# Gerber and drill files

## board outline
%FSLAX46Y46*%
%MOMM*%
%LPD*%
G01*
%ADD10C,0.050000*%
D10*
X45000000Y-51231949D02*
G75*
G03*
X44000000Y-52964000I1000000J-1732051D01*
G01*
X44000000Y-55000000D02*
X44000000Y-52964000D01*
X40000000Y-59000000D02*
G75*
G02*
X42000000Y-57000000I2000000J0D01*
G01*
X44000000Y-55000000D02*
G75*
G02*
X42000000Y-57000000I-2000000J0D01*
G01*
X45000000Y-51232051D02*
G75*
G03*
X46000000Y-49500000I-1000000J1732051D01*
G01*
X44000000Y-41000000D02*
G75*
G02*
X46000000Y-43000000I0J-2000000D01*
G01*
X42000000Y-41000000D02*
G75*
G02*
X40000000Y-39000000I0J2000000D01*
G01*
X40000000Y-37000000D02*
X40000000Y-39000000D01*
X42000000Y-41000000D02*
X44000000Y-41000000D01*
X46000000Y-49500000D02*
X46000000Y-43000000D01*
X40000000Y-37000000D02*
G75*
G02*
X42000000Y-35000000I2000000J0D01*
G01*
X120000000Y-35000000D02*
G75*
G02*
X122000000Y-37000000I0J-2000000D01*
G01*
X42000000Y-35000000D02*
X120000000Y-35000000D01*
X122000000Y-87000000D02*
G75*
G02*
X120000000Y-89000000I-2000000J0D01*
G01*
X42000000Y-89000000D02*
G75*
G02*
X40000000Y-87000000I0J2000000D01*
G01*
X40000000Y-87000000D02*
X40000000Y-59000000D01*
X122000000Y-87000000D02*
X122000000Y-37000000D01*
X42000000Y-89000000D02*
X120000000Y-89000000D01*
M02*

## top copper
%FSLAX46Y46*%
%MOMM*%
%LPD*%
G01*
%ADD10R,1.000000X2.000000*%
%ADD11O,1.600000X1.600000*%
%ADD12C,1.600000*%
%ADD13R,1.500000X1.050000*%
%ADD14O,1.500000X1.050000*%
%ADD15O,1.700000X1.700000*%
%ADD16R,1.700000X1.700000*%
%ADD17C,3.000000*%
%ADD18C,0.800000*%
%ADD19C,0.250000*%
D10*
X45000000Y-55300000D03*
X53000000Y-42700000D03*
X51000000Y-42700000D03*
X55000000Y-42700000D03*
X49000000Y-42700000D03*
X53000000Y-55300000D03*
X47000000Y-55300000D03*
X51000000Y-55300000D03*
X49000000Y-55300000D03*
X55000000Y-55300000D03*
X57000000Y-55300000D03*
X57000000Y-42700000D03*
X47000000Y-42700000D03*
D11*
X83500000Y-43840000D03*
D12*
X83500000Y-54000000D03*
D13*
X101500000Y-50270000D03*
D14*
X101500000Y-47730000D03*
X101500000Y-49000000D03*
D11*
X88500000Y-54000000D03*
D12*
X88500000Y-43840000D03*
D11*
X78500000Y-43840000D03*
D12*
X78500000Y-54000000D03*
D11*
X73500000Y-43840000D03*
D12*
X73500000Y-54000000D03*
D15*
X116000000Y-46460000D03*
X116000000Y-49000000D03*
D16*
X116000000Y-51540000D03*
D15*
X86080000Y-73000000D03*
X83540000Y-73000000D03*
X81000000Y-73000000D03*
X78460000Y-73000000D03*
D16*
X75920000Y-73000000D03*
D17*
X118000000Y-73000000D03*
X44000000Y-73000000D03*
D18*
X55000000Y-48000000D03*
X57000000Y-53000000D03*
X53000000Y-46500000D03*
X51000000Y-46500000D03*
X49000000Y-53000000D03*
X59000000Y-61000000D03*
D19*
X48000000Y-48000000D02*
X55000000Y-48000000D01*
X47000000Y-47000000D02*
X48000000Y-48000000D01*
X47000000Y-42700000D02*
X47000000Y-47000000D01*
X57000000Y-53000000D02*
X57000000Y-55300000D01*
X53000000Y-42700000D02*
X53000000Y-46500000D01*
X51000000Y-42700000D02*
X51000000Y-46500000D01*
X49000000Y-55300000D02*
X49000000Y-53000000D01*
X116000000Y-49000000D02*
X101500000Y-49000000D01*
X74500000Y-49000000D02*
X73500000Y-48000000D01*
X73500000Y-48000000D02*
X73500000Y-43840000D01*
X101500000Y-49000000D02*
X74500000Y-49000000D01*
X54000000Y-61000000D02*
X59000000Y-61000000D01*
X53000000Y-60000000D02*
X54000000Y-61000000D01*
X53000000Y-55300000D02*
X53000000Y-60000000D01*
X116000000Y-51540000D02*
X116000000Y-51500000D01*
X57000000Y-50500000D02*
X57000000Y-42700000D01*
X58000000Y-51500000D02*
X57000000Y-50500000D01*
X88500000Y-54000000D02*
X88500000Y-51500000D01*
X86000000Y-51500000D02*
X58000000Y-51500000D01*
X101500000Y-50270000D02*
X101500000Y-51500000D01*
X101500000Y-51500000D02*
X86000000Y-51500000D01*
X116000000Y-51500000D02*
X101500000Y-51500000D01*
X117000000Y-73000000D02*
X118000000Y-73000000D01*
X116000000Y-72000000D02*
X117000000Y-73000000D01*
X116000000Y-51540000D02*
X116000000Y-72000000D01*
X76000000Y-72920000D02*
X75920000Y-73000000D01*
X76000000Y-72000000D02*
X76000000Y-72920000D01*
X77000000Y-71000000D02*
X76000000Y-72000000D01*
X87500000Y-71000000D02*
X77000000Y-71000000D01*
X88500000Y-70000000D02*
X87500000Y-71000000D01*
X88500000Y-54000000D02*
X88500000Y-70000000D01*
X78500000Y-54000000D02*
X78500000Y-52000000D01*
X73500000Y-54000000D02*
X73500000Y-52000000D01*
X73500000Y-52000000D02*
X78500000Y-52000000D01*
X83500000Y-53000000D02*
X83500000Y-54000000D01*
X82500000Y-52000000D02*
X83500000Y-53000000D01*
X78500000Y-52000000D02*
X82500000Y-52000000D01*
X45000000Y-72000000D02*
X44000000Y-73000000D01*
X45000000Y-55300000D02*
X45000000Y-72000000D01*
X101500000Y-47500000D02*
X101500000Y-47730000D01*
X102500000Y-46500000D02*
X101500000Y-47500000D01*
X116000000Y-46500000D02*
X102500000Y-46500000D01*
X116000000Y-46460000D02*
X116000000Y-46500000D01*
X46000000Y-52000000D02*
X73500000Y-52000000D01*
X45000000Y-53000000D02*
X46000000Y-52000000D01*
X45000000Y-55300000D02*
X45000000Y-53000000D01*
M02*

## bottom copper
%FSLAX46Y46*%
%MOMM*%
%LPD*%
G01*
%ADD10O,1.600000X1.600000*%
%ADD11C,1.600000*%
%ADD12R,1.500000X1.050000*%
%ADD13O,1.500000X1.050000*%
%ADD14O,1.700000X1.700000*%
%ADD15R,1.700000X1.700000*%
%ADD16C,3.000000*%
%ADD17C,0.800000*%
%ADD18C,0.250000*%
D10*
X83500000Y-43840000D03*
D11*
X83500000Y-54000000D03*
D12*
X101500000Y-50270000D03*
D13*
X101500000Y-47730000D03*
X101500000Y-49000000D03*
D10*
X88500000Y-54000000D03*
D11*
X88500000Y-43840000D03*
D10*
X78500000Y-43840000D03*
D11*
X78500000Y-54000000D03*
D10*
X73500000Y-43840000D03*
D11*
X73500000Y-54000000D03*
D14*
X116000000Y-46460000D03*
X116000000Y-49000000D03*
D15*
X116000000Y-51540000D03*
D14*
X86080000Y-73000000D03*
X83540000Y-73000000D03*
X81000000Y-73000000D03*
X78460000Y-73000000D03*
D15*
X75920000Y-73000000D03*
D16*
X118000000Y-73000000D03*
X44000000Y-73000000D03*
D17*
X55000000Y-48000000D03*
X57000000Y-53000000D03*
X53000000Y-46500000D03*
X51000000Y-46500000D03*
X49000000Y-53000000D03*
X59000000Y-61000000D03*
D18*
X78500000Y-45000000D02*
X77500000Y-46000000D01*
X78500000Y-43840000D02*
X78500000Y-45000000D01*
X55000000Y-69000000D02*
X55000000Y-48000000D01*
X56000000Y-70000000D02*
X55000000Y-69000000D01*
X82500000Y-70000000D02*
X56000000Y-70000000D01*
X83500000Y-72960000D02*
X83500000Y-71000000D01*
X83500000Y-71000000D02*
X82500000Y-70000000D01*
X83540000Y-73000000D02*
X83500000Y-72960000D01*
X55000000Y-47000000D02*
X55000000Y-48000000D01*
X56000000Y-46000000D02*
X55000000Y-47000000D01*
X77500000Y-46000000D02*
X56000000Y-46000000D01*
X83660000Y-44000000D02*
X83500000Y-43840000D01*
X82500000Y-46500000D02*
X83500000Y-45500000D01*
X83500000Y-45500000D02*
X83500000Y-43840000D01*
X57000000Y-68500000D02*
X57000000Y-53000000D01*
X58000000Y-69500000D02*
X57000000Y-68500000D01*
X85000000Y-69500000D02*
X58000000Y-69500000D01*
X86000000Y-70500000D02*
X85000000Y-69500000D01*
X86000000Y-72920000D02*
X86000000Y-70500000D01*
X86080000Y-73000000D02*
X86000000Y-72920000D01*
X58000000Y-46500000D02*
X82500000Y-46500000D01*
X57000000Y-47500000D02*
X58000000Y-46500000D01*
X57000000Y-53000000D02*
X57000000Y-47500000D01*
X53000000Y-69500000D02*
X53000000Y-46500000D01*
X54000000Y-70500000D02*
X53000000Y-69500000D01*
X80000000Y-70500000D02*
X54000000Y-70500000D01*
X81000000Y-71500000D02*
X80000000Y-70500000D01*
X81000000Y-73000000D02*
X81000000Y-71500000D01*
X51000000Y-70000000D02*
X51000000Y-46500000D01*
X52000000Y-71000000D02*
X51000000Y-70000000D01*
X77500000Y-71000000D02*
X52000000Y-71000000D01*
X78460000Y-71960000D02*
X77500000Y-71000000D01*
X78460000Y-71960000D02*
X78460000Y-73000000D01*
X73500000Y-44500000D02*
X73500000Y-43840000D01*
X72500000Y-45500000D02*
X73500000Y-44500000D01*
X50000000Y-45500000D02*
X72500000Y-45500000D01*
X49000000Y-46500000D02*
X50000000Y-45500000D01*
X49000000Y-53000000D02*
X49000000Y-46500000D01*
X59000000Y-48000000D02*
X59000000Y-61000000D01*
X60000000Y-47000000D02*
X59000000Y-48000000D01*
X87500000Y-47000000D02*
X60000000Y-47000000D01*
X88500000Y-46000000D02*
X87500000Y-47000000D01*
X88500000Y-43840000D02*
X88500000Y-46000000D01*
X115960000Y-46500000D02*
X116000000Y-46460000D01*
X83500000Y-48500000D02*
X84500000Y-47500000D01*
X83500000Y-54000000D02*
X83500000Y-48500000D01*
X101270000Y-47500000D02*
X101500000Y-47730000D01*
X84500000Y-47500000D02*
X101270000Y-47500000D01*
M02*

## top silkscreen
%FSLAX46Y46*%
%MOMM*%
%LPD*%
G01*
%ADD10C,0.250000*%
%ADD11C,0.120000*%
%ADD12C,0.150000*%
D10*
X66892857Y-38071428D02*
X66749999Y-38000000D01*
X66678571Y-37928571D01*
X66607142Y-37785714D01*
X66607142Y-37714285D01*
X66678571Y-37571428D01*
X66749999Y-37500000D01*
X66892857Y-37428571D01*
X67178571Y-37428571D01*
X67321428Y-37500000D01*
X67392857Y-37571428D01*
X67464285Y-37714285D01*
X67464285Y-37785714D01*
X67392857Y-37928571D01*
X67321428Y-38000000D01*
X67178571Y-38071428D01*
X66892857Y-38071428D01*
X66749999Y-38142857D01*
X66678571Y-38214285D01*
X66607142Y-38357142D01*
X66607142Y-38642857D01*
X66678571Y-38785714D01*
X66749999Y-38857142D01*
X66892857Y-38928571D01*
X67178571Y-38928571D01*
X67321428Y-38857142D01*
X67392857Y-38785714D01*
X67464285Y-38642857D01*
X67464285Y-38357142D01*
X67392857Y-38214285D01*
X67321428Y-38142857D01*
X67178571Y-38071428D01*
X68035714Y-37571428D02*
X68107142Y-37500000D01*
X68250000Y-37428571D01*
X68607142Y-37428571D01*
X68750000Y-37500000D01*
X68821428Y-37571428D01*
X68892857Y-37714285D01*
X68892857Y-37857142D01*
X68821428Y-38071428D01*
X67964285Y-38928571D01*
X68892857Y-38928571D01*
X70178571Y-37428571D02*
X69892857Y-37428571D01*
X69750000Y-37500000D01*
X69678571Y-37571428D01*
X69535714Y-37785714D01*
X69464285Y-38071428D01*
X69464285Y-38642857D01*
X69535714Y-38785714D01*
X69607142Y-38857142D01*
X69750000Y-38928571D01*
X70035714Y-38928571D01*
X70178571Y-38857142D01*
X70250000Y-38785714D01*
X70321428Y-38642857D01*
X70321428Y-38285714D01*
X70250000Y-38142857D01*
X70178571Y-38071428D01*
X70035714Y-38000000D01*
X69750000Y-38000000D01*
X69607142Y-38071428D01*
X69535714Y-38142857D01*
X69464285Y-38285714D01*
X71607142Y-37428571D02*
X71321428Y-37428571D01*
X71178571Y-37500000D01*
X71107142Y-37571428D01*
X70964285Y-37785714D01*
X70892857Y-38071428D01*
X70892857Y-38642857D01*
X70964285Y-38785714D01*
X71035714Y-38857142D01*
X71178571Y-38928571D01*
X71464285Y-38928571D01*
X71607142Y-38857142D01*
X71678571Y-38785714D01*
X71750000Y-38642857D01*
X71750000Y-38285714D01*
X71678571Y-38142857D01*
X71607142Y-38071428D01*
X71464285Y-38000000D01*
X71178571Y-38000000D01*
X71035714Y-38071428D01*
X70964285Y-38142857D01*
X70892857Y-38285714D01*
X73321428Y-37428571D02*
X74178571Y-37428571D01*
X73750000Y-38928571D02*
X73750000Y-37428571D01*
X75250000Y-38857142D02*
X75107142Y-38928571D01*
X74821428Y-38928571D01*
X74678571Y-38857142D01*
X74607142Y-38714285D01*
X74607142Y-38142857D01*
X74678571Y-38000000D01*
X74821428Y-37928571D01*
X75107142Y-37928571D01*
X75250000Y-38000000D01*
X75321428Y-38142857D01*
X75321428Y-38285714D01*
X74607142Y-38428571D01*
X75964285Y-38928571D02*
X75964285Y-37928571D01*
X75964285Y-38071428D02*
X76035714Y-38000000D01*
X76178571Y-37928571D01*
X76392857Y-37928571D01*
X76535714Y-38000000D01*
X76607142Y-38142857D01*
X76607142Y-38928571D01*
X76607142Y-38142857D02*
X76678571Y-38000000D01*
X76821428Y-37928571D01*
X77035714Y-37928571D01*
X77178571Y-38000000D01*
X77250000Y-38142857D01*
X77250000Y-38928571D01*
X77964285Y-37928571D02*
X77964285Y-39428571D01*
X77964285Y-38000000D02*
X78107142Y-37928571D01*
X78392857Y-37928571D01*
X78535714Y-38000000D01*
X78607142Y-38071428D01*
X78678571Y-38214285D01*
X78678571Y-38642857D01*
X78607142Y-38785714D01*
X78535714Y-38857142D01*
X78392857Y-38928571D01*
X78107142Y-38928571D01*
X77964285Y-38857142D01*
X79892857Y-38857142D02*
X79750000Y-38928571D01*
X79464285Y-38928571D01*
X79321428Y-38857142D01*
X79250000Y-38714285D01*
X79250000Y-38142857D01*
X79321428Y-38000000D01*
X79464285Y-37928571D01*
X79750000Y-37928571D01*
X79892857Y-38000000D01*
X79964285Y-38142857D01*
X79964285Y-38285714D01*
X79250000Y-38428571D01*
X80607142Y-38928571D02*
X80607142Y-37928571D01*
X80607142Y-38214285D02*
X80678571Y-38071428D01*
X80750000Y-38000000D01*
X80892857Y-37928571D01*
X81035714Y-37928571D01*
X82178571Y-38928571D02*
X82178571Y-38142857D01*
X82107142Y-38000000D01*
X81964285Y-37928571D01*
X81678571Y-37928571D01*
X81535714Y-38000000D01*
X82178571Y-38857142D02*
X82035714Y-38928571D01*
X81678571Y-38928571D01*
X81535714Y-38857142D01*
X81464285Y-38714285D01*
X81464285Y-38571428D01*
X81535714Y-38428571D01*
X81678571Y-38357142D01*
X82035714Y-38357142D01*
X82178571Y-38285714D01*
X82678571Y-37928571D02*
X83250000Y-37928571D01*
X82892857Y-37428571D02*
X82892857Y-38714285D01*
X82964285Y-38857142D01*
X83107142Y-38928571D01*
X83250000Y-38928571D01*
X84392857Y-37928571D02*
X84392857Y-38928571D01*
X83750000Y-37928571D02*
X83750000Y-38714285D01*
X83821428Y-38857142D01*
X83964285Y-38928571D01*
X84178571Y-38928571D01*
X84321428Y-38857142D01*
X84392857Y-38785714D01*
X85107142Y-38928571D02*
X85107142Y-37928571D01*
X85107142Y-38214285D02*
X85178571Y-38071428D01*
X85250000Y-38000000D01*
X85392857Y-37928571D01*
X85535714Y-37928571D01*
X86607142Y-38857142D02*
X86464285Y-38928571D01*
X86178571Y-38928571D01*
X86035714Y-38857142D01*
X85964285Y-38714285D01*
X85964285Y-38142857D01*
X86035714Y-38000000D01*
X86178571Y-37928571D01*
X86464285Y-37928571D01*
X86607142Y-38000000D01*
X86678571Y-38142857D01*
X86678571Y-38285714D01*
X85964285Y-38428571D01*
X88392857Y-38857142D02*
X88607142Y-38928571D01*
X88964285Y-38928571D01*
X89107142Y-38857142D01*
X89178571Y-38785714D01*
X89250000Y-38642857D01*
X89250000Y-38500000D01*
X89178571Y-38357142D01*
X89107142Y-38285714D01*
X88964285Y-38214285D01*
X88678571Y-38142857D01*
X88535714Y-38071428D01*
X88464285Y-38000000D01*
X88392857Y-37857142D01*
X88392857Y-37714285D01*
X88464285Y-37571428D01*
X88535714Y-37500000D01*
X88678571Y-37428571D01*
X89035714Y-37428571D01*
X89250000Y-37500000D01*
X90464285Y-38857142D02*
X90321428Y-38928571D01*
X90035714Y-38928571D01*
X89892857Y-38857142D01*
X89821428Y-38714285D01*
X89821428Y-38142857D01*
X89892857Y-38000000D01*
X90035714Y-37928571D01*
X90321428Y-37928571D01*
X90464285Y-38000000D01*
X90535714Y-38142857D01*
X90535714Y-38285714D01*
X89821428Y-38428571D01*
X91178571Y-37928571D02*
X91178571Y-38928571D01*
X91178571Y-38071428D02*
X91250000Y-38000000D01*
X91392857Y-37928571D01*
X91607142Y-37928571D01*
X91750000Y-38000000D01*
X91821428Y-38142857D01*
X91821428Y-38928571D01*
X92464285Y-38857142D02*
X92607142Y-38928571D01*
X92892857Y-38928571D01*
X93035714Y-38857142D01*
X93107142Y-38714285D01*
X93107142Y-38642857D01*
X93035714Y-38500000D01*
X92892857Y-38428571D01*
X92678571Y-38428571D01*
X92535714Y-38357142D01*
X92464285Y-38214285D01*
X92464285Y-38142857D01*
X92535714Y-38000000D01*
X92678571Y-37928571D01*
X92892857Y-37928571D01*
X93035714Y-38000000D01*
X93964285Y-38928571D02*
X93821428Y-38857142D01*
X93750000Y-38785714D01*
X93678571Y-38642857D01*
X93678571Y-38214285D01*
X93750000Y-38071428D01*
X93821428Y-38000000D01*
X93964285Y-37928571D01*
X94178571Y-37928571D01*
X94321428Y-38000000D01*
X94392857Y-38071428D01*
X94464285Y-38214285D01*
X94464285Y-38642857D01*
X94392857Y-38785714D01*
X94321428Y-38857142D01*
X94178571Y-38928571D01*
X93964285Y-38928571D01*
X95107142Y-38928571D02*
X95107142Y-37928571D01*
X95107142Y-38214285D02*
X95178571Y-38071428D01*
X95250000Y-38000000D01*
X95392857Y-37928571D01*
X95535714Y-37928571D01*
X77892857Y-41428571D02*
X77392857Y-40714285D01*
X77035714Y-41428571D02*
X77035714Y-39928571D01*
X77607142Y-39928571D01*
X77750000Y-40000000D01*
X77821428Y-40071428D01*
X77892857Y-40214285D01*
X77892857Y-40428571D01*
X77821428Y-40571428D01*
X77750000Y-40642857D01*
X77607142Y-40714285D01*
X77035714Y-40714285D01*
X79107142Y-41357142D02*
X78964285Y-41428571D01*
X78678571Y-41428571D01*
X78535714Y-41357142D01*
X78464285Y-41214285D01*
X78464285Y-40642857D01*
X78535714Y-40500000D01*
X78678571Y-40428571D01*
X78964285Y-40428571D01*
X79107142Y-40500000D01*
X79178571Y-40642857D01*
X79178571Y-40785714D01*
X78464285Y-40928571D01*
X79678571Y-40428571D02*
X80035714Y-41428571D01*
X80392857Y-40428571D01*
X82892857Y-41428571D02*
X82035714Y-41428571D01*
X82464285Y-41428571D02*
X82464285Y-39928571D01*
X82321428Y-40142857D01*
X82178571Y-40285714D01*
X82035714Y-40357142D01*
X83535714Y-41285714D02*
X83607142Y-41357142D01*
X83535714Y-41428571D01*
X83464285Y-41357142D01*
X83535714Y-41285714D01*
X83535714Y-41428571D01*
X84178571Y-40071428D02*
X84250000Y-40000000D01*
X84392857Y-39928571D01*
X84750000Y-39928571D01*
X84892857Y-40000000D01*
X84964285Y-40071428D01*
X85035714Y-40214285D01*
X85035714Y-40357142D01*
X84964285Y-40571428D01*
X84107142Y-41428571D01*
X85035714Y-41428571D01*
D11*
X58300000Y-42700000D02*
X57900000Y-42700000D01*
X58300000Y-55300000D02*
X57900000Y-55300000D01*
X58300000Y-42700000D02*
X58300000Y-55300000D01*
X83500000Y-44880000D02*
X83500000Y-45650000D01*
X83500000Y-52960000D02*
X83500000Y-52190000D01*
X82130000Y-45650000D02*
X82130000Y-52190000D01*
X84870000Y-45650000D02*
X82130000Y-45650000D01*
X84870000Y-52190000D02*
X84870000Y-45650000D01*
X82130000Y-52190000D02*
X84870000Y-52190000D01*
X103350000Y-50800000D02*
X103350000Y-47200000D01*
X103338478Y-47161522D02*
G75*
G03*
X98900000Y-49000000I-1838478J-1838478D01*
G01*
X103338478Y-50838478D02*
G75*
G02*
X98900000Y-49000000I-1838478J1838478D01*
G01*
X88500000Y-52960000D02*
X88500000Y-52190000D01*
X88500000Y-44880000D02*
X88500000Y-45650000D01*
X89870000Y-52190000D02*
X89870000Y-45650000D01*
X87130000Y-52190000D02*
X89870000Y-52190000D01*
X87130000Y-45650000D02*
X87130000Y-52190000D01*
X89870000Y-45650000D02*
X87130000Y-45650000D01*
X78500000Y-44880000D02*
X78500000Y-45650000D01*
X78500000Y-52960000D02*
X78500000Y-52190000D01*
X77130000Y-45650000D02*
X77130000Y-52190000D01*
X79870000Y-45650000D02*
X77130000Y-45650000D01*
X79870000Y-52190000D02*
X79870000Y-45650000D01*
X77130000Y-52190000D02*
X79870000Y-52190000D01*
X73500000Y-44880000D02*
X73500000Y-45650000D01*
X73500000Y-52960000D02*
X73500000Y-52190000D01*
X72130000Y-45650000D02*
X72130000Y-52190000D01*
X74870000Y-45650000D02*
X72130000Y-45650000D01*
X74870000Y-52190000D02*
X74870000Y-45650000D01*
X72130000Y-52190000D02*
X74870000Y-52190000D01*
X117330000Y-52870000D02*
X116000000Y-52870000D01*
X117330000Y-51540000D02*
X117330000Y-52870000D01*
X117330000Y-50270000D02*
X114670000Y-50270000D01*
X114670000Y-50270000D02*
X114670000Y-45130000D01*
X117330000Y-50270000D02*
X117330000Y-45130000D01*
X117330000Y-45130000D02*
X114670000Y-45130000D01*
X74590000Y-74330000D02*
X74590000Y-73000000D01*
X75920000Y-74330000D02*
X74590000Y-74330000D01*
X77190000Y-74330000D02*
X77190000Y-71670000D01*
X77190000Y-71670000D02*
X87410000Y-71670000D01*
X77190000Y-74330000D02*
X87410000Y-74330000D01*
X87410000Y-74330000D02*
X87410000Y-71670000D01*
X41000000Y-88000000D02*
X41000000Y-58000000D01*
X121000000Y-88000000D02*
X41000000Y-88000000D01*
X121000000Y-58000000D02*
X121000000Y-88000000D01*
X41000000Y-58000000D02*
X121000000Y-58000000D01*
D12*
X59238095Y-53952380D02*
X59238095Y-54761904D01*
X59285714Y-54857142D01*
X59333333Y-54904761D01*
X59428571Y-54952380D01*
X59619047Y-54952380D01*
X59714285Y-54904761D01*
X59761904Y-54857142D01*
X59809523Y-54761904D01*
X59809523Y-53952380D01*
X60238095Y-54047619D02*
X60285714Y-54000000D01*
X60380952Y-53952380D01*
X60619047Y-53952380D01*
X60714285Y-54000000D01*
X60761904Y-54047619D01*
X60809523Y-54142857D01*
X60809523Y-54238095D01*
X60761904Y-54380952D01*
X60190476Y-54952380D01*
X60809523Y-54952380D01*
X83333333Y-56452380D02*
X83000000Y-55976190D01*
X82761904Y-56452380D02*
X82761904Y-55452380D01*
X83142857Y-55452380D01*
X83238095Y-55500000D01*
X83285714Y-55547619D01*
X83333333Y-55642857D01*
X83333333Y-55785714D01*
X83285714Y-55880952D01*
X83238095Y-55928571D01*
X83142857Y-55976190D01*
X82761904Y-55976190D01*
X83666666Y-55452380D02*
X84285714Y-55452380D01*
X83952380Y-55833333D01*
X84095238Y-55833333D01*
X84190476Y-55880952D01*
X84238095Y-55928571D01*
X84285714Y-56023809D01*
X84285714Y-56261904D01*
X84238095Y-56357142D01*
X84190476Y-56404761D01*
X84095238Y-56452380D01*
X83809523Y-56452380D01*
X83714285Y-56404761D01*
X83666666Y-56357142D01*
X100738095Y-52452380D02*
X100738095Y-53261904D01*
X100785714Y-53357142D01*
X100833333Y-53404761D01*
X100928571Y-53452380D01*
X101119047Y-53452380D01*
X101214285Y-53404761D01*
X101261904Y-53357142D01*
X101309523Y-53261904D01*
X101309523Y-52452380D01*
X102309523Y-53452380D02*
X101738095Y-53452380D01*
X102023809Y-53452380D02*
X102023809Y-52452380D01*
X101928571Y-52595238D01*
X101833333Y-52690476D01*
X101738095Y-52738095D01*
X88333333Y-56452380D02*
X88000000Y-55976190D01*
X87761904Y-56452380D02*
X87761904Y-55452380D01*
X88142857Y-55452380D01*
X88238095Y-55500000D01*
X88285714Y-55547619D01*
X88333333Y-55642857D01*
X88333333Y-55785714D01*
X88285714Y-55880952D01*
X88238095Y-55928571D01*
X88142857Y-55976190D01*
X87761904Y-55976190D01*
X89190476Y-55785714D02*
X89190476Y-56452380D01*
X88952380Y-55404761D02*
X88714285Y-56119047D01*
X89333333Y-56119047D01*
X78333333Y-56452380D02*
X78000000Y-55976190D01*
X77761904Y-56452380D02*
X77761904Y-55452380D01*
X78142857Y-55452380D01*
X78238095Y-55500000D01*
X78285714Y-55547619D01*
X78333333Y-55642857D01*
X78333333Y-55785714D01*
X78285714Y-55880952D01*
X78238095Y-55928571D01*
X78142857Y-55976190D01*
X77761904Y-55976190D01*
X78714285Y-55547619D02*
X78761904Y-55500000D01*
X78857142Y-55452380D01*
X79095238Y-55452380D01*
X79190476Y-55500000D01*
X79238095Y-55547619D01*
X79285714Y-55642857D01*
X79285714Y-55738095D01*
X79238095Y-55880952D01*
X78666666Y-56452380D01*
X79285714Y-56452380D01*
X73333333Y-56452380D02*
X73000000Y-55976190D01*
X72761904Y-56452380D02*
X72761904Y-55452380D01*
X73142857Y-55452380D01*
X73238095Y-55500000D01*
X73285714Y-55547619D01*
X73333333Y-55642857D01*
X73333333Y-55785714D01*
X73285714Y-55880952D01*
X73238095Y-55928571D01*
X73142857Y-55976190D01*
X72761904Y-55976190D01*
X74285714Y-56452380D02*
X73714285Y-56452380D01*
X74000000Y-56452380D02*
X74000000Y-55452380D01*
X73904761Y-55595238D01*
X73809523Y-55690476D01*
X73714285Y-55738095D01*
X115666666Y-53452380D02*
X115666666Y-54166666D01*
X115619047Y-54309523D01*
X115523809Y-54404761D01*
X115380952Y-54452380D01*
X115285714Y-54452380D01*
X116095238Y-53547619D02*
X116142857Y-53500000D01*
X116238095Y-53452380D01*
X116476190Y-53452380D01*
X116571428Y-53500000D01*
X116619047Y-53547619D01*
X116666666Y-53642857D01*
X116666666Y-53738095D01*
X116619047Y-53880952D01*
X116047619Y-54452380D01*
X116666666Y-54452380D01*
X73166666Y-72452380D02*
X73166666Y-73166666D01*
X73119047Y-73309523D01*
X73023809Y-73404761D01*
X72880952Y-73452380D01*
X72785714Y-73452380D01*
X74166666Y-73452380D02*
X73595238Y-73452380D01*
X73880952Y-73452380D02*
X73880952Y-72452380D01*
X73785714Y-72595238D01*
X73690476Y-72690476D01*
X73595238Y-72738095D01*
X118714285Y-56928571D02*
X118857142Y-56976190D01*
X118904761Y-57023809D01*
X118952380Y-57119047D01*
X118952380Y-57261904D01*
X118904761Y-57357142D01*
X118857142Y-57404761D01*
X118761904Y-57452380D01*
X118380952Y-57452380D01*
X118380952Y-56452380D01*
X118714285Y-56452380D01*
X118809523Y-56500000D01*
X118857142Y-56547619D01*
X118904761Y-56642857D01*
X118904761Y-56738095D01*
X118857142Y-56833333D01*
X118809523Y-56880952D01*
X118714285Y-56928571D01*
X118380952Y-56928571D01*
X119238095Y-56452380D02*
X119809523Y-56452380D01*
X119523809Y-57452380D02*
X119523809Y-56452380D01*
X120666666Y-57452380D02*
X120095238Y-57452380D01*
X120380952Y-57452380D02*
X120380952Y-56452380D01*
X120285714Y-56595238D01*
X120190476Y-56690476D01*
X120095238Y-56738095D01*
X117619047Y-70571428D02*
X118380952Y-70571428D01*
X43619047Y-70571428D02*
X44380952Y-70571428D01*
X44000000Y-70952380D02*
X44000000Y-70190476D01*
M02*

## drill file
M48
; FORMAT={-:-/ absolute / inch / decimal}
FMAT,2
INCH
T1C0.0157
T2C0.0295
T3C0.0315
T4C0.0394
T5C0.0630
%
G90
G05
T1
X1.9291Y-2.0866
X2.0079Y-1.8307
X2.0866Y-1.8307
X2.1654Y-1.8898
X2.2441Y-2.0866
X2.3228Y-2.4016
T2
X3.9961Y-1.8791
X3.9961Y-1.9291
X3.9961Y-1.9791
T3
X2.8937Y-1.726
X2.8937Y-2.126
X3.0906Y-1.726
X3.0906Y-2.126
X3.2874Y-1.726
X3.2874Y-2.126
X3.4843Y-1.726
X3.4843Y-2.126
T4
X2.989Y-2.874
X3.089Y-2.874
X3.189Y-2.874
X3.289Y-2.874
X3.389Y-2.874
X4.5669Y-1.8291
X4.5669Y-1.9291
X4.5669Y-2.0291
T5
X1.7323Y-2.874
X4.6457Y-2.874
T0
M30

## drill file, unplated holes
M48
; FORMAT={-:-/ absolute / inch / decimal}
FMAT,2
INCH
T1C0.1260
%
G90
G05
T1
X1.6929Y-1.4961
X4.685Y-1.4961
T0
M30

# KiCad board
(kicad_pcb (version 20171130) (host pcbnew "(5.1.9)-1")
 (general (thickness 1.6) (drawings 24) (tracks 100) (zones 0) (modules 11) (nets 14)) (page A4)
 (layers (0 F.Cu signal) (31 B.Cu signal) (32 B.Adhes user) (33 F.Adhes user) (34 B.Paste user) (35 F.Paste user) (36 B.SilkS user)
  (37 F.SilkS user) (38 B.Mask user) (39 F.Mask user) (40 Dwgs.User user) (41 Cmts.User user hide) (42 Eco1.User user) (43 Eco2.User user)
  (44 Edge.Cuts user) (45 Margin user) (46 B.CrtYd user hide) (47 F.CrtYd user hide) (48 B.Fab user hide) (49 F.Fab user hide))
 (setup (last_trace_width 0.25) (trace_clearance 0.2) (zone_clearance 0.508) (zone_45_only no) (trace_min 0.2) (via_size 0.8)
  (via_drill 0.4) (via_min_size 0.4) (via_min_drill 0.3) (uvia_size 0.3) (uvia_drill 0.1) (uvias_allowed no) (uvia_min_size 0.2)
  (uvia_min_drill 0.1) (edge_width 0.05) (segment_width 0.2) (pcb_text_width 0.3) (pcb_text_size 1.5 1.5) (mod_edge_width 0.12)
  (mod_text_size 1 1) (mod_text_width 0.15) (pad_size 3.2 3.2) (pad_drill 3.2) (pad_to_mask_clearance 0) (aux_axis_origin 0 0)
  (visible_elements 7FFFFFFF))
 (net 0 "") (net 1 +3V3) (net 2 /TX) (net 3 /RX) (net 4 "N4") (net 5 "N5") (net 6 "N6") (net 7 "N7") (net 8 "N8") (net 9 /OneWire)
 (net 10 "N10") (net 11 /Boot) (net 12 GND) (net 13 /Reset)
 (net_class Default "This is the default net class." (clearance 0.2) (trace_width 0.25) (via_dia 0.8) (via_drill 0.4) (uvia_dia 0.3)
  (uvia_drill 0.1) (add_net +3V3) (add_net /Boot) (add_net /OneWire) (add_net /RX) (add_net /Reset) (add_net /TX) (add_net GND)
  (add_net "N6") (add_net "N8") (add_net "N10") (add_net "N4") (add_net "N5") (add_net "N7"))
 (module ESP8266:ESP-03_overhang (layer F.Cu) (at 51 49 90)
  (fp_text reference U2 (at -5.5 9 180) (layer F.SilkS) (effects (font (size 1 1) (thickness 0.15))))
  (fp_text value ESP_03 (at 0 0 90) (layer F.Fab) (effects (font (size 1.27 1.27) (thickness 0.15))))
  (fp_line (start 6.3 7.3) (end 6.3 6.9) (layer F.SilkS) (width 0.12))
  (fp_line (start -6.3 7.3) (end -6.3 6.9) (layer F.SilkS) (width 0.12))
  (fp_line (start 6.3 7.3) (end -6.3 7.3) (layer F.SilkS) (width 0.12))
  (pad 8 smd rect (at -6.3 -6 90) (size 2 1) (layers F.Cu F.Paste F.Mask) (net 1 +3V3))
  (pad 3 smd rect (at 6.3 2 90) (size 2 1) (layers F.Cu F.Paste F.Mask) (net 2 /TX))
  (pad 4 smd rect (at 6.3 0 90) (size 2 1) (layers F.Cu F.Paste F.Mask) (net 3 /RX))
  (pad 2 smd rect (at 6.3 4 90) (size 2 1) (layers F.Cu F.Paste F.Mask) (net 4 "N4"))
  (pad 5 smd rect (at 6.3 -2 90) (size 2 1) (layers F.Cu F.Paste F.Mask) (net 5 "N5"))
  (pad 12 smd rect (at -6.3 2 90) (size 2 1) (layers F.Cu F.Paste F.Mask) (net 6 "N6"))
  (pad 9 smd rect (at -6.3 -4 90) (size 2 1) (layers F.Cu F.Paste F.Mask) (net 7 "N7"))
  (pad 11 smd rect (at -6.3 0 90) (size 2 1) (layers F.Cu F.Paste F.Mask) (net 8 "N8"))
  (pad 10 smd rect (at -6.3 -2 90) (size 2 1) (layers F.Cu F.Paste F.Mask) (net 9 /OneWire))
  (pad 13 smd rect (at -6.3 4 90) (size 2 1) (layers F.Cu F.Paste F.Mask) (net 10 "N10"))
  (pad 14 smd rect (at -6.3 6 90) (size 2 1) (layers F.Cu F.Paste F.Mask) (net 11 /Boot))
  (pad 1 smd rect (at 6.3 6 90) (size 2 1) (layers F.Cu F.Paste F.Mask) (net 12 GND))
  (pad 6 smd rect (at 6.3 -4 90) (size 2 1) (layers F.Cu F.Paste F.Mask) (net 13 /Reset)))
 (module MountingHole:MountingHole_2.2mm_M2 (layer F.Cu) (at 119 38)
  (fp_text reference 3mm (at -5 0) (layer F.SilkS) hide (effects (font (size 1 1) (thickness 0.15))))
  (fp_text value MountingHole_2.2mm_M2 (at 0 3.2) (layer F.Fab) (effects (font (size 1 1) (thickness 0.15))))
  (pad "" np_thru_hole circle (at 0 0) (size 3.2 3.2) (drill 3.2) (layers *.Cu *.Mask)))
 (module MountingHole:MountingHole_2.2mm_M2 (layer F.Cu) (at 43 38)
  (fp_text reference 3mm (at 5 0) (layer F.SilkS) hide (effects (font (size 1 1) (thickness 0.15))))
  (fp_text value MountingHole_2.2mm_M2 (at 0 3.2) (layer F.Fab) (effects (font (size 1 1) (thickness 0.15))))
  (pad "" np_thru_hole circle (at 0 0) (size 3.2 3.2) (drill 3.2) (layers *.Cu *.Mask)))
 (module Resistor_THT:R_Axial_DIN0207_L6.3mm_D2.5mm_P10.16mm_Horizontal (layer F.Cu) (at 83.5 54 90)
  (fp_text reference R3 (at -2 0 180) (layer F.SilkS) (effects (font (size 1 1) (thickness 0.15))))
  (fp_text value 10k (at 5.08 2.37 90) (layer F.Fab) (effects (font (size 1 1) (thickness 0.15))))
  (fp_line (start 9.12 0) (end 8.35 0) (layer F.SilkS) (width 0.12))
  (fp_line (start 1.04 0) (end 1.81 0) (layer F.SilkS) (width 0.12))
  (fp_line (start 8.35 -1.37) (end 1.81 -1.37) (layer F.SilkS) (width 0.12))
  (fp_line (start 8.35 1.37) (end 8.35 -1.37) (layer F.SilkS) (width 0.12))
  (fp_line (start 1.81 1.37) (end 8.35 1.37) (layer F.SilkS) (width 0.12))
  (fp_line (start 1.81 -1.37) (end 1.81 1.37) (layer F.SilkS) (width 0.12))
  (pad 2 thru_hole oval (at 10.16 0 90) (size 1.6 1.6) (drill 0.8) (layers *.Cu *.Mask) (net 11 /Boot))
  (pad 1 thru_hole circle (at 0 0 90) (size 1.6 1.6) (drill 0.8) (layers *.Cu *.Mask) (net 1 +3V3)))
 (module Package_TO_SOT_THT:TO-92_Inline (layer F.Cu) (at 101.5 50.27 90)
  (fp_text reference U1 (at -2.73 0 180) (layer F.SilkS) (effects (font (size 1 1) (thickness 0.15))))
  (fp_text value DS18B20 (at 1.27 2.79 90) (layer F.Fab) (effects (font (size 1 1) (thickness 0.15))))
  (fp_line (start -0.53 1.85) (end 3.07 1.85) (layer F.SilkS) (width 0.12))
  (fp_arc (start 1.27 0) (end 1.27 -2.6) (angle 135) (layer F.SilkS) (width 0.12))
  (fp_arc (start 1.27 0) (end 1.27 -2.6) (angle -135) (layer F.SilkS) (width 0.12))
  (pad 1 thru_hole rect (at 0 0 90) (size 1.05 1.5) (drill 0.75) (layers *.Cu *.Mask) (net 12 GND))
  (pad 3 thru_hole oval (at 2.54 0 90) (size 1.05 1.5) (drill 0.75) (layers *.Cu *.Mask) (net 1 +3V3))
  (pad 2 thru_hole oval (at 1.27 0 90) (size 1.05 1.5) (drill 0.75) (layers *.Cu *.Mask) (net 9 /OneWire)))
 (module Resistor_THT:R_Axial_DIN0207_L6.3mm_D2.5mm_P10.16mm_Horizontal (layer F.Cu) (at 88.5 43.84 270)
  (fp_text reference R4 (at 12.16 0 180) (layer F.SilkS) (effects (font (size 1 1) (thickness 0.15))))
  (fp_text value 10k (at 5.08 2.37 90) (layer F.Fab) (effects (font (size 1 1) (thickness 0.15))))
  (fp_line (start 9.12 0) (end 8.35 0) (layer F.SilkS) (width 0.12))
  (fp_line (start 1.04 0) (end 1.81 0) (layer F.SilkS) (width 0.12))
  (fp_line (start 8.35 -1.37) (end 1.81 -1.37) (layer F.SilkS) (width 0.12))
  (fp_line (start 8.35 1.37) (end 8.35 -1.37) (layer F.SilkS) (width 0.12))
  (fp_line (start 1.81 1.37) (end 8.35 1.37) (layer F.SilkS) (width 0.12))
  (fp_line (start 1.81 -1.37) (end 1.81 1.37) (layer F.SilkS) (width 0.12))
  (pad 2 thru_hole oval (at 10.16 0 270) (size 1.6 1.6) (drill 0.8) (layers *.Cu *.Mask) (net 12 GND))
  (pad 1 thru_hole circle (at 0 0 270) (size 1.6 1.6) (drill 0.8) (layers *.Cu *.Mask) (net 6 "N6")))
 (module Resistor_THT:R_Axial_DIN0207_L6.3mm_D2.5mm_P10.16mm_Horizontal (layer F.Cu) (at 78.5 54 90)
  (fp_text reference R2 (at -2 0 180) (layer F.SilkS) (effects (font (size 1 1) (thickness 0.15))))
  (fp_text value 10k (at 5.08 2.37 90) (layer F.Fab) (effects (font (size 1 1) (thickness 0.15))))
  (fp_line (start 9.12 0) (end 8.35 0) (layer F.SilkS) (width 0.12))
  (fp_line (start 1.04 0) (end 1.81 0) (layer F.SilkS) (width 0.12))
  (fp_line (start 8.35 -1.37) (end 1.81 -1.37) (layer F.SilkS) (width 0.12))
  (fp_line (start 8.35 1.37) (end 8.35 -1.37) (layer F.SilkS) (width 0.12))
  (fp_line (start 1.81 1.37) (end 8.35 1.37) (layer F.SilkS) (width 0.12))
  (fp_line (start 1.81 -1.37) (end 1.81 1.37) (layer F.SilkS) (width 0.12))
  (pad 2 thru_hole oval (at 10.16 0 90) (size 1.6 1.6) (drill 0.8) (layers *.Cu *.Mask) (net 13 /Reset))
  (pad 1 thru_hole circle (at 0 0 90) (size 1.6 1.6) (drill 0.8) (layers *.Cu *.Mask) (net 1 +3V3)))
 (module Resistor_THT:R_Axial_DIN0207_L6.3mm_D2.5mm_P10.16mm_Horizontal (layer F.Cu) (at 73.5 54 90)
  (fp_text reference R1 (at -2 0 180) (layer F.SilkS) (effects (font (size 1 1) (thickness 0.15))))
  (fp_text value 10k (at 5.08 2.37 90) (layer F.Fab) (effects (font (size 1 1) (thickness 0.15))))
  (fp_line (start 9.12 0) (end 8.35 0) (layer F.SilkS) (width 0.12))
  (fp_line (start 1.04 0) (end 1.81 0) (layer F.SilkS) (width 0.12))
  (fp_line (start 8.35 -1.37) (end 1.81 -1.37) (layer F.SilkS) (width 0.12))
  (fp_line (start 8.35 1.37) (end 8.35 -1.37) (layer F.SilkS) (width 0.12))
  (fp_line (start 1.81 1.37) (end 8.35 1.37) (layer F.SilkS) (width 0.12))
  (fp_line (start 1.81 -1.37) (end 1.81 1.37) (layer F.SilkS) (width 0.12))
  (pad 2 thru_hole oval (at 10.16 0 90) (size 1.6 1.6) (drill 0.8) (layers *.Cu *.Mask) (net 9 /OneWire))
  (pad 1 thru_hole circle (at 0 0 90) (size 1.6 1.6) (drill 0.8) (layers *.Cu *.Mask) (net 1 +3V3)))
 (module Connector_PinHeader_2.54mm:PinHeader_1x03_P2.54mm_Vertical (layer F.Cu) (at 116 51.54 180)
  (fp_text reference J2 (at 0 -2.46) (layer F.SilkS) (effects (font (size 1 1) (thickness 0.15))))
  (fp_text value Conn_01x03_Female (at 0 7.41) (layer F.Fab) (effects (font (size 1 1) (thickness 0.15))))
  (fp_line (start -1.33 -1.33) (end 0 -1.33) (layer F.SilkS) (width 0.12))
  (fp_line (start -1.33 0) (end -1.33 -1.33) (layer F.SilkS) (width 0.12))
  (fp_line (start -1.33 1.27) (end 1.33 1.27) (layer F.SilkS) (width 0.12))
  (fp_line (start 1.33 1.27) (end 1.33 6.41) (layer F.SilkS) (width 0.12))
  (fp_line (start -1.33 1.27) (end -1.33 6.41) (layer F.SilkS) (width 0.12))
  (fp_line (start -1.33 6.41) (end 1.33 6.41) (layer F.SilkS) (width 0.12))
  (pad 3 thru_hole oval (at 0 5.08 180) (size 1.7 1.7) (drill 1) (layers *.Cu *.Mask) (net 1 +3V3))
  (pad 2 thru_hole oval (at 0 2.54 180) (size 1.7 1.7) (drill 1) (layers *.Cu *.Mask) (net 9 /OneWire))
  (pad 1 thru_hole rect (at 0 0 180) (size 1.7 1.7) (drill 1) (layers *.Cu *.Mask) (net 12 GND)))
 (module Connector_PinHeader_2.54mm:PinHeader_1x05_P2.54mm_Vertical (layer F.Cu) (at 75.92 73 90)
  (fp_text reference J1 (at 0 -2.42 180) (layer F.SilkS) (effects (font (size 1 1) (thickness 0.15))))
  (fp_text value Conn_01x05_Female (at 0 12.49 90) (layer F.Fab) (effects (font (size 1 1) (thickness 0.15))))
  (fp_line (start -1.33 -1.33) (end 0 -1.33) (layer F.SilkS) (width 0.12))
  (fp_line (start -1.33 0) (end -1.33 -1.33) (layer F.SilkS) (width 0.12))
  (fp_line (start -1.33 1.27) (end 1.33 1.27) (layer F.SilkS) (width 0.12))
  (fp_line (start 1.33 1.27) (end 1.33 11.49) (layer F.SilkS) (width 0.12))
  (fp_line (start -1.33 1.27) (end -1.33 11.49) (layer F.SilkS) (width 0.12))
  (fp_line (start -1.33 11.49) (end 1.33 11.49) (layer F.SilkS) (width 0.12))
  (pad 5 thru_hole oval (at 0 10.16 90) (size 1.7 1.7) (drill 1) (layers *.Cu *.Mask) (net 11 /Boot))
  (pad 4 thru_hole oval (at 0 7.62 90) (size 1.7 1.7) (drill 1) (layers *.Cu *.Mask) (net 13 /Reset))
  (pad 3 thru_hole oval (at 0 5.08 90) (size 1.7 1.7) (drill 1) (layers *.Cu *.Mask) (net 2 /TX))
  (pad 2 thru_hole oval (at 0 2.54 90) (size 1.7 1.7) (drill 1) (layers *.Cu *.Mask) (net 3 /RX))
  (pad 1 thru_hole rect (at 0 0 90) (size 1.7 1.7) (drill 1) (layers *.Cu *.Mask) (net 12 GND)))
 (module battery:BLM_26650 (layer F.Cu) (at 81 73)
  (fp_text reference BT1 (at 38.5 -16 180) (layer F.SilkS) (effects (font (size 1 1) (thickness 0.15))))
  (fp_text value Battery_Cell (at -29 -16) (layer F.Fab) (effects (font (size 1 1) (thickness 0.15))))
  (fp_line (start -40 15) (end -40 -15) (layer F.SilkS) (width 0.12))
  (fp_line (start 40 15) (end -40 15) (layer F.SilkS) (width 0.12))
  (fp_line (start 40 -15) (end 40 15) (layer F.SilkS) (width 0.12))
  (fp_line (start -40 -15) (end 40 -15) (layer F.SilkS) (width 0.12))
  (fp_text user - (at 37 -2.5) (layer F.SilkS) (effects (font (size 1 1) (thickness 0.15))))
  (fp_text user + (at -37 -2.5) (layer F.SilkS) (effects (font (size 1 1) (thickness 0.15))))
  (pad 2 thru_hole circle (at 37 0) (size 3 3) (drill 1.6) (layers *.Cu *.Mask) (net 12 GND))
  (pad 1 thru_hole circle (at -37 0) (size 3 3) (drill 1.6) (layers *.Cu *.Mask) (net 1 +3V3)))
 (gr_arc (start 46 52.964) (end 44 52.964) (angle 60) (layer Edge.Cuts) (width 0.05))
 (gr_line (start 44 55) (end 44 52.964) (layer Edge.Cuts) (width 0.05))
 (gr_arc (start 42 59) (end 42 57) (angle -90) (layer Edge.Cuts) (width 0.05))
 (gr_arc (start 42 55) (end 42 57) (angle -90) (layer Edge.Cuts) (width 0.05))
 (gr_arc (start 44 49.5) (end 46 49.5) (angle 60.00000276) (layer Edge.Cuts) (width 0.05))
 (gr_arc (start 44 43) (end 46 43) (angle -90) (layer Edge.Cuts) (width 0.05))
 (gr_arc (start 42 39) (end 40 39) (angle -90) (layer Edge.Cuts) (width 0.05))
 (gr_line (start 40 37) (end 40 39) (layer Edge.Cuts) (width 0.05))
 (gr_line (start 42 41) (end 44 41) (layer Edge.Cuts) (width 0.05))
 (gr_line (start 46 49.5) (end 46 43) (layer Edge.Cuts) (width 0.05))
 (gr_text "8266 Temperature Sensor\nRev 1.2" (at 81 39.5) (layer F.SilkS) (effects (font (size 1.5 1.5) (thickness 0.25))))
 (gr_arc (start 42 37) (end 42 35) (angle -90) (layer Edge.Cuts) (width 0.05))
 (gr_arc (start 120 37) (end 122 37) (angle -90) (layer Edge.Cuts) (width 0.05))
 (gr_line (start 42 35) (end 120 35) (layer Edge.Cuts) (width 0.05))
 (gr_arc (start 120 87) (end 120 89) (angle -90) (layer Edge.Cuts) (width 0.05))
 (gr_arc (start 42 87) (end 40 87) (angle -90) (layer Edge.Cuts) (width 0.05))
 (gr_line (start 40 87) (end 40 59) (layer Edge.Cuts) (width 0.05))
 (gr_line (start 122 87) (end 122 37) (layer Edge.Cuts) (width 0.05))
 (gr_line (start 42 89) (end 120 89) (layer Edge.Cuts) (width 0.05))
 (via (at 55 48) (size 0.8) (drill 0.4) (layers F.Cu B.Cu) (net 13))
 (segment (start 48 48) (end 55 48) (width 0.25) (layer F.Cu) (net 13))
 (segment (start 47 47) (end 48 48) (width 0.25) (layer F.Cu) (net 13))
 (segment (start 47 42.7) (end 47 47) (width 0.25) (layer F.Cu) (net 13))
 (segment (start 78.5 45) (end 77.5 46) (width 0.25) (layer B.Cu) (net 13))
 (segment (start 78.5 43.84) (end 78.5 45) (width 0.25) (layer B.Cu) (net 13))
 (segment (start 55 69) (end 55 48) (width 0.25) (layer B.Cu) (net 13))
 (segment (start 56 70) (end 55 69) (width 0.25) (layer B.Cu) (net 13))
 (segment (start 82.5 70) (end 56 70) (width 0.25) (layer B.Cu) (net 13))
 (segment (start 83.5 72.96) (end 83.5 71) (width 0.25) (layer B.Cu) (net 13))
 (segment (start 83.5 71) (end 82.5 70) (width 0.25) (layer B.Cu) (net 13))
 (segment (start 83.54 73) (end 83.5 72.96) (width 0.25) (layer B.Cu) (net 13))
 (segment (start 55 47) (end 55 48) (width 0.25) (layer B.Cu) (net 13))
 (segment (start 56 46) (end 55 47) (width 0.25) (layer B.Cu) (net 13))
 (segment (start 77.5 46) (end 56 46) (width 0.25) (layer B.Cu) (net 13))
 (segment (start 83.66 44) (end 83.5 43.84) (width 0.25) (layer B.Cu) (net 11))
 (via (at 57 53) (size 0.8) (drill 0.4) (layers F.Cu B.Cu) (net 11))
 (segment (start 57 53) (end 57 55.3) (width 0.25) (layer F.Cu) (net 11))
 (segment (start 82.5 46.5) (end 83.5 45.5) (width 0.25) (layer B.Cu) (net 11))
 (segment (start 83.5 45.5) (end 83.5 43.84) (width 0.25) (layer B.Cu) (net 11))
 (segment (start 57 68.5) (end 57 53) (width 0.25) (layer B.Cu) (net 11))
 (segment (start 58 69.5) (end 57 68.5) (width 0.25) (layer B.Cu) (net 11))
 (segment (start 85 69.5) (end 58 69.5) (width 0.25) (layer B.Cu) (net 11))
 (segment (start 86 70.5) (end 85 69.5) (width 0.25) (layer B.Cu) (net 11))
 (segment (start 86 72.92) (end 86 70.5) (width 0.25) (layer B.Cu) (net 11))
 (segment (start 86.08 73) (end 86 72.92) (width 0.25) (layer B.Cu) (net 11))
 (segment (start 58 46.5) (end 82.5 46.5) (width 0.25) (layer B.Cu) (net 11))
 (segment (start 57 47.5) (end 58 46.5) (width 0.25) (layer B.Cu) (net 11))
 (segment (start 57 53) (end 57 47.5) (width 0.25) (layer B.Cu) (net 11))
 (via (at 53 46.5) (size 0.8) (drill 0.4) (layers F.Cu B.Cu) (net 2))
 (segment (start 53 42.7) (end 53 46.5) (width 0.25) (layer F.Cu) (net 2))
 (segment (start 53 69.5) (end 53 46.5) (width 0.25) (layer B.Cu) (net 2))
 (segment (start 54 70.5) (end 53 69.5) (width 0.25) (layer B.Cu) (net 2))
 (segment (start 80 70.5) (end 54 70.5) (width 0.25) (layer B.Cu) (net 2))
 (segment (start 81 71.5) (end 80 70.5) (width 0.25) (layer B.Cu) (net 2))
 (segment (start 81 73) (end 81 71.5) (width 0.25) (layer B.Cu) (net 2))
 (via (at 51 46.5) (size 0.8) (drill 0.4) (layers F.Cu B.Cu) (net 3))
 (segment (start 51 42.7) (end 51 46.5) (width 0.25) (layer F.Cu) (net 3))
 (segment (start 51 70) (end 51 46.5) (width 0.25) (layer B.Cu) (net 3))
 (segment (start 52 71) (end 51 70) (width 0.25) (layer B.Cu) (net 3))
 (segment (start 77.5 71) (end 52 71) (width 0.25) (layer B.Cu) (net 3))
 (segment (start 78.46 71.96) (end 77.5 71) (width 0.25) (layer B.Cu) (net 3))
 (segment (start 78.46 71.96) (end 78.46 73) (width 0.25) (layer B.Cu) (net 3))
 (via (at 49 53) (size 0.8) (drill 0.4) (layers F.Cu B.Cu) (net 9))
 (segment (start 49 55.3) (end 49 53) (width 0.25) (layer F.Cu) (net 9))
 (segment (start 116 49) (end 101.5 49) (width 0.25) (layer F.Cu) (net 9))
 (segment (start 74.5 49) (end 73.5 48) (width 0.25) (layer F.Cu) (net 9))
 (segment (start 73.5 48) (end 73.5 43.84) (width 0.25) (layer F.Cu) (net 9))
 (segment (start 73.5 44.5) (end 73.5 43.84) (width 0.25) (layer B.Cu) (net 9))
 (segment (start 72.5 45.5) (end 73.5 44.5) (width 0.25) (layer B.Cu) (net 9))
 (segment (start 101.5 49) (end 74.5 49) (width 0.25) (layer F.Cu) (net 9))
 (segment (start 50 45.5) (end 72.5 45.5) (width 0.25) (layer B.Cu) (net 9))
 (segment (start 49 46.5) (end 50 45.5) (width 0.25) (layer B.Cu) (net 9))
 (segment (start 49 53) (end 49 46.5) (width 0.25) (layer B.Cu) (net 9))
 (via (at 59 61) (size 0.8) (drill 0.4) (layers F.Cu B.Cu) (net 6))
 (segment (start 54 61) (end 59 61) (width 0.25) (layer F.Cu) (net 6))
 (segment (start 53 60) (end 54 61) (width 0.25) (layer F.Cu) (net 6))
 (segment (start 53 55.3) (end 53 60) (width 0.25) (layer F.Cu) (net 6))
 (segment (start 59 48) (end 59 61) (width 0.25) (layer B.Cu) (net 6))
 (segment (start 60 47) (end 59 48) (width 0.25) (layer B.Cu) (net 6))
 (segment (start 87.5 47) (end 60 47) (width 0.25) (layer B.Cu) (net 6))
 (segment (start 88.5 46) (end 87.5 47) (width 0.25) (layer B.Cu) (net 6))
 (segment (start 88.5 43.84) (end 88.5 46) (width 0.25) (layer B.Cu) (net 6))
 (segment (start 116 51.54) (end 116 51.5) (width 0.25) (layer F.Cu) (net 12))
 (segment (start 57 50.5) (end 57 42.7) (width 0.25) (layer F.Cu) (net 12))
 (segment (start 58 51.5) (end 57 50.5) (width 0.25) (layer F.Cu) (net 12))
 (segment (start 88.5 54) (end 88.5 51.5) (width 0.25) (layer F.Cu) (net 12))
 (segment (start 86 51.5) (end 58 51.5) (width 0.25) (layer F.Cu) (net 12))
 (segment (start 101.5 50.27) (end 101.5 51.5) (width 0.25) (layer F.Cu) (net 12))
 (segment (start 101.5 51.5) (end 86 51.5) (width 0.25) (layer F.Cu) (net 12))
 (segment (start 116 51.5) (end 101.5 51.5) (width 0.25) (layer F.Cu) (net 12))
 (segment (start 117 73) (end 118 73) (width 0.25) (layer F.Cu) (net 12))
 (segment (start 116 72) (end 117 73) (width 0.25) (layer F.Cu) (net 12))
 (segment (start 116 51.54) (end 116 72) (width 0.25) (layer F.Cu) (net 12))
 (segment (start 76 72.92) (end 75.92 73) (width 0.25) (layer F.Cu) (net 12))
 (segment (start 76 72) (end 76 72.92) (width 0.25) (layer F.Cu) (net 12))
 (segment (start 77 71) (end 76 72) (width 0.25) (layer F.Cu) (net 12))
 (segment (start 87.5 71) (end 77 71) (width 0.25) (layer F.Cu) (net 12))
 (segment (start 88.5 70) (end 87.5 71) (width 0.25) (layer F.Cu) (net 12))
 (segment (start 88.5 54) (end 88.5 70) (width 0.25) (layer F.Cu) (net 12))
 (segment (start 78.5 54) (end 78.5 52) (width 0.25) (layer F.Cu) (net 1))
 (segment (start 73.5 54) (end 73.5 52) (width 0.25) (layer F.Cu) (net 1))
 (segment (start 73.5 52) (end 78.5 52) (width 0.25) (layer F.Cu) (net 1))
 (segment (start 115.96 46.5) (end 116 46.46) (width 0.25) (layer B.Cu) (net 1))
 (segment (start 83.5 53) (end 83.5 54) (width 0.25) (layer F.Cu) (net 1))
 (segment (start 82.5 52) (end 83.5 53) (width 0.25) (layer F.Cu) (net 1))
 (segment (start 78.5 52) (end 82.5 52) (width 0.25) (layer F.Cu) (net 1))
 (segment (start 45 72) (end 44 73) (width 0.25) (layer F.Cu) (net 1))
 (segment (start 45 55.3) (end 45 72) (width 0.25) (layer F.Cu) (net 1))
 (segment (start 101.5 47.5) (end 101.5 47.73) (width 0.25) (layer F.Cu) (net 1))
 (segment (start 102.5 46.5) (end 101.5 47.5) (width 0.25) (layer F.Cu) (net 1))
 (segment (start 116 46.5) (end 102.5 46.5) (width 0.25) (layer F.Cu) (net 1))
 (segment (start 116 46.46) (end 116 46.5) (width 0.25) (layer F.Cu) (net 1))
 (segment (start 83.5 48.5) (end 84.5 47.5) (width 0.25) (layer B.Cu) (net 1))
 (segment (start 83.5 54) (end 83.5 48.5) (width 0.25) (layer B.Cu) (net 1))
 (segment (start 46 52) (end 73.5 52) (width 0.25) (layer F.Cu) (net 1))
 (segment (start 45 53) (end 46 52) (width 0.25) (layer F.Cu) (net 1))
 (segment (start 45 55.3) (end 45 53) (width 0.25) (layer F.Cu) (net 1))
 (segment (start 101.27 47.5) (end 101.5 47.73) (width 0.25) (layer B.Cu) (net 1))
 (segment (start 84.5 47.5) (end 101.27 47.5) (width 0.25) (layer B.Cu) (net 1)))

